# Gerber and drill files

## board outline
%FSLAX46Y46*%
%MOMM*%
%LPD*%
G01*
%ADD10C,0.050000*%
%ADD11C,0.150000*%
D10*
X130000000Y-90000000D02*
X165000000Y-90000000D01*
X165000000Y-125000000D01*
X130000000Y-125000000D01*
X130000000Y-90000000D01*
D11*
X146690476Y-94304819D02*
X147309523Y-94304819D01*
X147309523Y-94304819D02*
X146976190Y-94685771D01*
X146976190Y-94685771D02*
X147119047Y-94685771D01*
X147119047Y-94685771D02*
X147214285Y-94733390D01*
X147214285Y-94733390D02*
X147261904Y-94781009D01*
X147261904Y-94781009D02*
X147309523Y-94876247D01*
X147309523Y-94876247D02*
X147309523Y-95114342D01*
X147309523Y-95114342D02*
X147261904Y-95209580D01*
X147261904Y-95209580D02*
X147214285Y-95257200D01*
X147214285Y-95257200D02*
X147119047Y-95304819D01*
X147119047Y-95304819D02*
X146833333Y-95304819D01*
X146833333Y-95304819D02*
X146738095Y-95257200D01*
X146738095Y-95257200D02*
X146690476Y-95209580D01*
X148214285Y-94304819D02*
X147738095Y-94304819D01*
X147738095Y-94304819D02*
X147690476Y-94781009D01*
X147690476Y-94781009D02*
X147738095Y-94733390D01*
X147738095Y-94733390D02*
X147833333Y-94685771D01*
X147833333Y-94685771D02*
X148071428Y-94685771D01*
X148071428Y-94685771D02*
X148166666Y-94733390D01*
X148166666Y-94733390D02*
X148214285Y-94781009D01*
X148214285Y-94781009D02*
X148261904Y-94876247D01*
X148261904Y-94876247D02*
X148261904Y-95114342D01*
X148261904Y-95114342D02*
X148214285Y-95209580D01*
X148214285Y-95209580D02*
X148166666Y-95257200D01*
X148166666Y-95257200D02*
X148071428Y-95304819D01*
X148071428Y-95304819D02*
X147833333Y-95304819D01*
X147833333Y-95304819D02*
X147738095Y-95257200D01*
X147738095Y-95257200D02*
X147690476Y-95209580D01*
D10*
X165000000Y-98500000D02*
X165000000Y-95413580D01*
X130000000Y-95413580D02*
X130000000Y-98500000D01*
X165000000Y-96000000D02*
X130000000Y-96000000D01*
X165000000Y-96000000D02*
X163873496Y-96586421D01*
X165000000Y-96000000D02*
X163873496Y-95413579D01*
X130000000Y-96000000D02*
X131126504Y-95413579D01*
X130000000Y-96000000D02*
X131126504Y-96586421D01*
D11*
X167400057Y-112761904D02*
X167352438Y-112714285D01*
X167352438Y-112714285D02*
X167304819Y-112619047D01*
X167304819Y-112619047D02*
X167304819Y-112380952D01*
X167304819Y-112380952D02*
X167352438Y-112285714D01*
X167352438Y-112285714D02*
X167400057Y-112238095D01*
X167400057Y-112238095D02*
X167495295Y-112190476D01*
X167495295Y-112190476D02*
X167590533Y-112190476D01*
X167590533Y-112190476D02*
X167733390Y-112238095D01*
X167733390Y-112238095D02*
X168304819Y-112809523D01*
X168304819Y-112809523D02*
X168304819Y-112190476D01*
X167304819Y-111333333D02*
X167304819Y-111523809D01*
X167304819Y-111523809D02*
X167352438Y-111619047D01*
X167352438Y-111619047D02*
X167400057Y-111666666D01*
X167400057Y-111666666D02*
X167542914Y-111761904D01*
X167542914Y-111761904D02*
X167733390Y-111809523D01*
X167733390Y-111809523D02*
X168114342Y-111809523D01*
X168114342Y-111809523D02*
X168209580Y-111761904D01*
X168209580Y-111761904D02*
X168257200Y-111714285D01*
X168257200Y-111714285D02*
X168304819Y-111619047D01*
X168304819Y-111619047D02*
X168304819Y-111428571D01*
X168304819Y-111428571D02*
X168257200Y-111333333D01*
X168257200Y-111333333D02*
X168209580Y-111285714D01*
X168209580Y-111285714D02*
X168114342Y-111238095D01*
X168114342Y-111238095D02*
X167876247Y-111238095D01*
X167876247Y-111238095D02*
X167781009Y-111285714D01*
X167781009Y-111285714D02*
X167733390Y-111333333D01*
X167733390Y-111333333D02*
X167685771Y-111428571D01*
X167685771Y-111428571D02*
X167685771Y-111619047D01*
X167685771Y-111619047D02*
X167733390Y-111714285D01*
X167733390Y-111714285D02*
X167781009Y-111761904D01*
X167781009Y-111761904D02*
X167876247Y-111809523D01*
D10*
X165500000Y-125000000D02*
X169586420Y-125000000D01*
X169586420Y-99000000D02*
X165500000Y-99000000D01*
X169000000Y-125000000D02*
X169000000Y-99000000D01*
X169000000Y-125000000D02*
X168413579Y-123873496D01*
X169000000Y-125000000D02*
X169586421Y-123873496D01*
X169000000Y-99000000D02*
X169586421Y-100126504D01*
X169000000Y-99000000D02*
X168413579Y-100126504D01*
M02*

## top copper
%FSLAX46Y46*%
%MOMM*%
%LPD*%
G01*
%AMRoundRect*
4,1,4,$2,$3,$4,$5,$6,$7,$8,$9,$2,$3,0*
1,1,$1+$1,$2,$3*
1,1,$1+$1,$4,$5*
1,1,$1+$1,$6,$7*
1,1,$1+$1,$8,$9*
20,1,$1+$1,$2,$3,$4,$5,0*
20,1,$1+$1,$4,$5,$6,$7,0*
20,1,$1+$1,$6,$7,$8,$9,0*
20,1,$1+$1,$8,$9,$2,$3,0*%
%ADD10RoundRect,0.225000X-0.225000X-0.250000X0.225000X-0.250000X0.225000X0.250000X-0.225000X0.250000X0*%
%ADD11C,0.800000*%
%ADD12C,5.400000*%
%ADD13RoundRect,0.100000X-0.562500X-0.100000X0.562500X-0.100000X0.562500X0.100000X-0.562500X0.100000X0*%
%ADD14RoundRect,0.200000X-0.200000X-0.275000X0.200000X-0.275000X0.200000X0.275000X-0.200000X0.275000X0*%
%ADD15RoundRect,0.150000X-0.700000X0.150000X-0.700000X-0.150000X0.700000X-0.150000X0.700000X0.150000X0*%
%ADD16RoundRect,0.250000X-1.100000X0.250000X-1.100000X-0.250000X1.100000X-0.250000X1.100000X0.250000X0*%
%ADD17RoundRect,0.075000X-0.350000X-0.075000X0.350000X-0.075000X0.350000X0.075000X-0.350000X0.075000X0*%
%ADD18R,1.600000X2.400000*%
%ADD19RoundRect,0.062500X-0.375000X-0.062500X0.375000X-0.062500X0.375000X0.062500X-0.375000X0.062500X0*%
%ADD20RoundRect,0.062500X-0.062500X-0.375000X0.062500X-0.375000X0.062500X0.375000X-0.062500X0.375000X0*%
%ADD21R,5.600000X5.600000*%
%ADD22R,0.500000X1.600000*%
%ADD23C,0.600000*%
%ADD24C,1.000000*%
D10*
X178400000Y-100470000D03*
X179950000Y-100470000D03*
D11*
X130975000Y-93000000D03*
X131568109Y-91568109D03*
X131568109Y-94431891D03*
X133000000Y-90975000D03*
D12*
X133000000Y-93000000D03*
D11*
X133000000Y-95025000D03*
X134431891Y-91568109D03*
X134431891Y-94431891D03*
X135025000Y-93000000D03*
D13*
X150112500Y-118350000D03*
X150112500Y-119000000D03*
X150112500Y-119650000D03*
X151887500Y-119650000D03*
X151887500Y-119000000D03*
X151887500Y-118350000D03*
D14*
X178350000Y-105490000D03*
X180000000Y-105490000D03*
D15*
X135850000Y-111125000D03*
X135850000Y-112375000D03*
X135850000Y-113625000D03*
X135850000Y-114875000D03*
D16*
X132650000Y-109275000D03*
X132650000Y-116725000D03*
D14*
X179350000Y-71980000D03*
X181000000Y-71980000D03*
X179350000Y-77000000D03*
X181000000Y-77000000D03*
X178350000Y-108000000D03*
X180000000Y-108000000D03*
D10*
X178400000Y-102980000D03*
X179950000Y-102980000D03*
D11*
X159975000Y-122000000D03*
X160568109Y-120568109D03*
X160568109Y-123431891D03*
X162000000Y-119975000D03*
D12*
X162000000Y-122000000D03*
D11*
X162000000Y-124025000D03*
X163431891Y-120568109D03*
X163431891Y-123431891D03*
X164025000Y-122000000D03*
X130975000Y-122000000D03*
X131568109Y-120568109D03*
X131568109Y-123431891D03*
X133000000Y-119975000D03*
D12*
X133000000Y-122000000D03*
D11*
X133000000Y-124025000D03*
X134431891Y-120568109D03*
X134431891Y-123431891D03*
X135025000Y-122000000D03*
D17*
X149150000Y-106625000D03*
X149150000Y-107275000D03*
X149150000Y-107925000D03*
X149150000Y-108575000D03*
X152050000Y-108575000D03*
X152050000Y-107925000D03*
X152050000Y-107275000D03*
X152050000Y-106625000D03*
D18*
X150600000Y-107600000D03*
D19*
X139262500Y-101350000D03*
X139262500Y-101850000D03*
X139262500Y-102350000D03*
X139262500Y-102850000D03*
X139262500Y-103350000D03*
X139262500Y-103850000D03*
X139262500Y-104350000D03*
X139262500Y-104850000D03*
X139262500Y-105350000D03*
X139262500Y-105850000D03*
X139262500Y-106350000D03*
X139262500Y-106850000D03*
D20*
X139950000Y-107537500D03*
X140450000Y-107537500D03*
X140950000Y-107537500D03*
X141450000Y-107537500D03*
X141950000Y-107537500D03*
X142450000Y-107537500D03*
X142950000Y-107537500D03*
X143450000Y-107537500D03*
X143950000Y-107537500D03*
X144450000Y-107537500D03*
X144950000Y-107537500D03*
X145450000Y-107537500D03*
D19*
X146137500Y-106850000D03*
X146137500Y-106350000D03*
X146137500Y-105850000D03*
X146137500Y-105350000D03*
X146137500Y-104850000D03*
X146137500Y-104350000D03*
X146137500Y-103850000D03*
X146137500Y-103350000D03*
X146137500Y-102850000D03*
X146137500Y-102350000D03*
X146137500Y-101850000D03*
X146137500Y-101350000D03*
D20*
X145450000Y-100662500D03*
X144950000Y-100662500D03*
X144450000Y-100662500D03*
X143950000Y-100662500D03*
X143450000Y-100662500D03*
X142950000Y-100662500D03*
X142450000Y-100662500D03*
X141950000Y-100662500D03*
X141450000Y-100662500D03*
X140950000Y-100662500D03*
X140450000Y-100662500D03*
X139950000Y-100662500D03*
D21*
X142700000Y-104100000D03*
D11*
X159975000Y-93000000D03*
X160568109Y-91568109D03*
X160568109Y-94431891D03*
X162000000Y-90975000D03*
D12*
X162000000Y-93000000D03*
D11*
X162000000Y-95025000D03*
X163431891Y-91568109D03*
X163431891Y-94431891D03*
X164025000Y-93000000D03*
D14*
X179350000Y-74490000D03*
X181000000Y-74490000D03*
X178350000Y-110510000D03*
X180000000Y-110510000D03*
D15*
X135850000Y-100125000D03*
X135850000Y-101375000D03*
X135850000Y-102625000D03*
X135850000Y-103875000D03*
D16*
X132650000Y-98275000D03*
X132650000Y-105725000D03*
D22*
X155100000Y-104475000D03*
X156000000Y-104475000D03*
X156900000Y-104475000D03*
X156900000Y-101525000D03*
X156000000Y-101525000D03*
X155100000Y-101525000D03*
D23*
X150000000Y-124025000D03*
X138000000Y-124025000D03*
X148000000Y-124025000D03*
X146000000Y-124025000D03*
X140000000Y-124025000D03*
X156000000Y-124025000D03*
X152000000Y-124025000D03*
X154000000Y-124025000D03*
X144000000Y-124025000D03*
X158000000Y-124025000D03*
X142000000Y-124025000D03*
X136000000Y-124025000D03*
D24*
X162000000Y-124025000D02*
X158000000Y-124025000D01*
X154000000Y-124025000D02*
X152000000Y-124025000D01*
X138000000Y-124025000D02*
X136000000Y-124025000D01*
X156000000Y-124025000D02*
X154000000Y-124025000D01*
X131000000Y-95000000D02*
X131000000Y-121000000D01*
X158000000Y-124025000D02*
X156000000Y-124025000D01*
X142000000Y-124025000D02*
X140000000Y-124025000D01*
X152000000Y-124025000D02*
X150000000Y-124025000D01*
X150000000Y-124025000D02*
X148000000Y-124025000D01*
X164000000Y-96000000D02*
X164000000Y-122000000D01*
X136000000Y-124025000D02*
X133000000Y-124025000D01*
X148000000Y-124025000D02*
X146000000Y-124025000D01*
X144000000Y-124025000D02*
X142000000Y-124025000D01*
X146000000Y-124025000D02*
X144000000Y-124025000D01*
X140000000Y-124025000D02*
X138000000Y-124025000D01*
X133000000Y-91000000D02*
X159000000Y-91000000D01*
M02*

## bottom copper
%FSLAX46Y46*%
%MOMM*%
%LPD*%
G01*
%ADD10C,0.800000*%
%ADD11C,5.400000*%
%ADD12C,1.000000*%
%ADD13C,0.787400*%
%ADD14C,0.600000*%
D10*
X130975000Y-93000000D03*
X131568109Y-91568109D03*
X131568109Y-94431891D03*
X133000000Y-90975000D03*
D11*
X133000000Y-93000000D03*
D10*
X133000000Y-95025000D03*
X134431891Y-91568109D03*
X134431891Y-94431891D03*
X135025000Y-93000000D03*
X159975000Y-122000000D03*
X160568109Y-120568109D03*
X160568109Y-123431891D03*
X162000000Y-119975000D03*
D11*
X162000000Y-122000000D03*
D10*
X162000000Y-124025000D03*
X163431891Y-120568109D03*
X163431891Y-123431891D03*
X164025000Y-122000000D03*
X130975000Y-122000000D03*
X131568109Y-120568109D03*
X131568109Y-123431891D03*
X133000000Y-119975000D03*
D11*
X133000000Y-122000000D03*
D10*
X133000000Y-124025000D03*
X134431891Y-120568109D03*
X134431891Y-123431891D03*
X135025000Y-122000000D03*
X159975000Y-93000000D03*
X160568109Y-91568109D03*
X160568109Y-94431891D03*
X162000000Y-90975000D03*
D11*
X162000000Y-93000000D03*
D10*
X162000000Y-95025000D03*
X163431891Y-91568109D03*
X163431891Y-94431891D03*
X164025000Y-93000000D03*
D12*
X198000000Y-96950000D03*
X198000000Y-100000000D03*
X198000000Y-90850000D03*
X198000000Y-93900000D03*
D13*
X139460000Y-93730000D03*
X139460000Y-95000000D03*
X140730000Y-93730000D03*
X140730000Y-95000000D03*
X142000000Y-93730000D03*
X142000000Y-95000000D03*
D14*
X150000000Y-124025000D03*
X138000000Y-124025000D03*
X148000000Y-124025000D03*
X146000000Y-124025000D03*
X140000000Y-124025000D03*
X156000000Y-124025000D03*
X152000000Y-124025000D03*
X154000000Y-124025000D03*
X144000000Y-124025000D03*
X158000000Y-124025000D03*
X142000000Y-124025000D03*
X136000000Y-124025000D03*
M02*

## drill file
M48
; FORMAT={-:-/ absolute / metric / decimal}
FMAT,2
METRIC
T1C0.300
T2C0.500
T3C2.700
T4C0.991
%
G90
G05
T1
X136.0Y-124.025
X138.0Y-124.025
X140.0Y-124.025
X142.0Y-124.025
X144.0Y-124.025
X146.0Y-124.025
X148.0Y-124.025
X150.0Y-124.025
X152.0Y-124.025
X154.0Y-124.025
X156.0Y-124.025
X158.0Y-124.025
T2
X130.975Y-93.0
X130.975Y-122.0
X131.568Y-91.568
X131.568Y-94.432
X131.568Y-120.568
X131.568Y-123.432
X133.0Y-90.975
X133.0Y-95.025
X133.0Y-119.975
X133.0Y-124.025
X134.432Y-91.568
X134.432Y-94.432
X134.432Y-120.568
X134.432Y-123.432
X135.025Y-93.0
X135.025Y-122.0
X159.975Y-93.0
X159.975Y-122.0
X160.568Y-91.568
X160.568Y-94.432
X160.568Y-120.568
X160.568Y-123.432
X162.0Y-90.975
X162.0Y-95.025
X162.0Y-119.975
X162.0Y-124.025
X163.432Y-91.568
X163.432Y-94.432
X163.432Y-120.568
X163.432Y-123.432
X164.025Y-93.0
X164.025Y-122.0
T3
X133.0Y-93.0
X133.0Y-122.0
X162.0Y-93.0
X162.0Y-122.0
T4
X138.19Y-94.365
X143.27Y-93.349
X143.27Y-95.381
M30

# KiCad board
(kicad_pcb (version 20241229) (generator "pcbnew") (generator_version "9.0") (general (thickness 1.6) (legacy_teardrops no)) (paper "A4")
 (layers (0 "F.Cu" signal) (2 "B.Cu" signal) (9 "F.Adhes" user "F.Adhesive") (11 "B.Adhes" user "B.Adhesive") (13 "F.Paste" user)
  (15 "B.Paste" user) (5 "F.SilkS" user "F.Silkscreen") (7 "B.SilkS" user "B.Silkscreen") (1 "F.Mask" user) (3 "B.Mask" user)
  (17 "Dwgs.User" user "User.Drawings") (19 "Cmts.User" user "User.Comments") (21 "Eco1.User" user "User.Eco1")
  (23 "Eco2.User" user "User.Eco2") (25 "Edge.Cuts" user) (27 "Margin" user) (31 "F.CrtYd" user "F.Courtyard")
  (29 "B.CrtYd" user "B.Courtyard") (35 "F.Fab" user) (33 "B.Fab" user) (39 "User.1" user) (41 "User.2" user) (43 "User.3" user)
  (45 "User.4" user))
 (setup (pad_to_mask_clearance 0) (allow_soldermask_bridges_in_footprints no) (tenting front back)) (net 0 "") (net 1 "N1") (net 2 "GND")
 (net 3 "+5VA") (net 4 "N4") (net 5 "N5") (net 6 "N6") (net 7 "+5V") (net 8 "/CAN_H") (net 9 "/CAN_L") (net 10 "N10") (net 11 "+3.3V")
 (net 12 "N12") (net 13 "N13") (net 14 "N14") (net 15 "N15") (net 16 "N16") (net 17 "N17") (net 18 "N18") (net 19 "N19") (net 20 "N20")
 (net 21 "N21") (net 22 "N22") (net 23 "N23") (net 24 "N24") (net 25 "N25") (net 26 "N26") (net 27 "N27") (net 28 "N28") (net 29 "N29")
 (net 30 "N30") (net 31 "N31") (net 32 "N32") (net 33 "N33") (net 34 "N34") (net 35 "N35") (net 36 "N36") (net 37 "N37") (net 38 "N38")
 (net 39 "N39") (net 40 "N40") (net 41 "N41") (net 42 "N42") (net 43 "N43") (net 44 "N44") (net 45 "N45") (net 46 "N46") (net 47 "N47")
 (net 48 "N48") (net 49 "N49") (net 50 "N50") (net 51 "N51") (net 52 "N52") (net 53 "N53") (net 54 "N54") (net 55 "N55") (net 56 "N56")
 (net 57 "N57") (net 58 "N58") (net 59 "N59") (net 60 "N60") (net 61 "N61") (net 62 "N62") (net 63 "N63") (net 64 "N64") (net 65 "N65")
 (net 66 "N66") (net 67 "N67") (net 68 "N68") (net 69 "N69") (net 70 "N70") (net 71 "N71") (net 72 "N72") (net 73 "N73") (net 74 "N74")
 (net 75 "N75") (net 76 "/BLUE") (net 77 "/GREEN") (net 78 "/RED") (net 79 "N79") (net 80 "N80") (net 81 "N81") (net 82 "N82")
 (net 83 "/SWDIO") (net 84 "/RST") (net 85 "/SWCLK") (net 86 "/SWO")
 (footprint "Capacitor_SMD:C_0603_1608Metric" (layer "F.Cu") (at 179.175 100.47)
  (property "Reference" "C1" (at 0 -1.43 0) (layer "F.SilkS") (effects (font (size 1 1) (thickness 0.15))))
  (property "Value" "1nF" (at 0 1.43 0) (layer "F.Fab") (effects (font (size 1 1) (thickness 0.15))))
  (pad "1" smd roundrect (at -0.775 0) (size 0.9 0.95) (layers "F.Cu" "F.Mask" "F.Paste") (roundrect_rratio 0.25) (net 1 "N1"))
  (pad "2" smd roundrect (at 0.775 0) (size 0.9 0.95) (layers "F.Cu" "F.Mask" "F.Paste") (roundrect_rratio 0.25) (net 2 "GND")))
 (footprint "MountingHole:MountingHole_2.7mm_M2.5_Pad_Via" (layer "F.Cu") (at 133 93)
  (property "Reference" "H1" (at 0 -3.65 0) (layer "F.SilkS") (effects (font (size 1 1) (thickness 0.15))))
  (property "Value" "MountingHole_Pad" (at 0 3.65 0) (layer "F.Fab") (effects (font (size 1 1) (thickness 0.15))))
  (pad "1" thru_hole circle (at -2.025 0) (size 0.8 0.8) (drill 0.5) (layers "*.Cu" "*.Mask") (remove_unused_layers no) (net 1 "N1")
   (zone_connect 2))
  (pad "1" thru_hole circle (at -1.431891 -1.431891) (size 0.8 0.8) (drill 0.5) (layers "*.Cu" "*.Mask") (remove_unused_layers no)
   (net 1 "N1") (zone_connect 2))
  (pad "1" thru_hole circle (at -1.431891 1.431891) (size 0.8 0.8) (drill 0.5) (layers "*.Cu" "*.Mask") (remove_unused_layers no)
   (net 1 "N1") (zone_connect 2))
  (pad "1" thru_hole circle (at 0 -2.025) (size 0.8 0.8) (drill 0.5) (layers "*.Cu" "*.Mask") (remove_unused_layers no) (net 1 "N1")
   (zone_connect 2))
  (pad "1" thru_hole circle (at 0 0) (size 5.4 5.4) (drill 2.7) (layers "*.Cu" "*.Mask") (remove_unused_layers no) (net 1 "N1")
   (zone_connect 2))
  (pad "1" thru_hole circle (at 0 2.025) (size 0.8 0.8) (drill 0.5) (layers "*.Cu" "*.Mask") (remove_unused_layers no) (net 1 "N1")
   (zone_connect 2))
  (pad "1" thru_hole circle (at 1.431891 -1.431891) (size 0.8 0.8) (drill 0.5) (layers "*.Cu" "*.Mask") (remove_unused_layers no)
   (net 1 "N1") (zone_connect 2))
  (pad "1" thru_hole circle (at 1.431891 1.431891) (size 0.8 0.8) (drill 0.5) (layers "*.Cu" "*.Mask") (remove_unused_layers no)
   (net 1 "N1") (zone_connect 2))
  (pad "1" thru_hole circle (at 2.025 0) (size 0.8 0.8) (drill 0.5) (layers "*.Cu" "*.Mask") (remove_unused_layers no) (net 1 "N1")
   (zone_connect 2)))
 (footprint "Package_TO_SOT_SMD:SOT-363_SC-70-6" (layer "F.Cu") (at 151 119)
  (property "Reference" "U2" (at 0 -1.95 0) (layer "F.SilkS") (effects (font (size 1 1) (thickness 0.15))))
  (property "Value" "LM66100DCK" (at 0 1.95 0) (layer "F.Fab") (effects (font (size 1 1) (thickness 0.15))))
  (pad "1" smd roundrect (at -0.8875 -0.65) (size 1.325 0.4) (layers "F.Cu" "F.Mask" "F.Paste") (roundrect_rratio 0.25) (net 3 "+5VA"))
  (pad "2" smd roundrect (at -0.8875 0) (size 1.325 0.4) (layers "F.Cu" "F.Mask" "F.Paste") (roundrect_rratio 0.25) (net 2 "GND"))
  (pad "3" smd roundrect (at -0.8875 0.65) (size 1.325 0.4) (layers "F.Cu" "F.Mask" "F.Paste") (roundrect_rratio 0.25) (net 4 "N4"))
  (pad "4" smd roundrect (at 0.8875 0.65) (size 1.325 0.4) (layers "F.Cu" "F.Mask" "F.Paste") (roundrect_rratio 0.25) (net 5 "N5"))
  (pad "5" smd roundrect (at 0.8875 0) (size 1.325 0.4) (layers "F.Cu" "F.Mask" "F.Paste") (roundrect_rratio 0.25) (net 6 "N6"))
  (pad "6" smd roundrect (at 0.8875 -0.65) (size 1.325 0.4) (layers "F.Cu" "F.Mask" "F.Paste") (roundrect_rratio 0.25) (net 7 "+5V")))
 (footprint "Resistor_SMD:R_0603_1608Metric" (layer "F.Cu") (at 179.175 105.49)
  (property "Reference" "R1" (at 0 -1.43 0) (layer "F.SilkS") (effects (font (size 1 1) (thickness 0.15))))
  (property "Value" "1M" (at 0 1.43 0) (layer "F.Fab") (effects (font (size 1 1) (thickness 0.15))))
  (pad "1" smd roundrect (at -0.825 0) (size 0.8 0.95) (layers "F.Cu" "F.Mask" "F.Paste") (roundrect_rratio 0.25) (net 1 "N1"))
  (pad "2" smd roundrect (at 0.825 0) (size 0.8 0.95) (layers "F.Cu" "F.Mask" "F.Paste") (roundrect_rratio 0.25) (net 2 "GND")))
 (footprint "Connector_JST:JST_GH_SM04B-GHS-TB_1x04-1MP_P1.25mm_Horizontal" (layer "F.Cu") (at 134 113 -90)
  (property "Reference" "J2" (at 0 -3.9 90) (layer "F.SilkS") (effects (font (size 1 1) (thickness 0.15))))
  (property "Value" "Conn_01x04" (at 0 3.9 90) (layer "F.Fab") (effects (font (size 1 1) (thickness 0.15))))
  (pad "1" smd roundrect (at -1.875 -1.85 270) (size 0.6 1.7) (layers "F.Cu" "F.Mask" "F.Paste") (roundrect_rratio 0.25) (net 3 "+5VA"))
  (pad "2" smd roundrect (at -0.625 -1.85 270) (size 0.6 1.7) (layers "F.Cu" "F.Mask" "F.Paste") (roundrect_rratio 0.25) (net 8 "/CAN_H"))
  (pad "3" smd roundrect (at 0.625 -1.85 270) (size 0.6 1.7) (layers "F.Cu" "F.Mask" "F.Paste") (roundrect_rratio 0.25) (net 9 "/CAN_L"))
  (pad "4" smd roundrect (at 1.875 -1.85 270) (size 0.6 1.7) (layers "F.Cu" "F.Mask" "F.Paste") (roundrect_rratio 0.25) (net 2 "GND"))
  (pad "MP" smd roundrect (at -3.725 1.35 270) (size 1 2.7) (layers "F.Cu" "F.Mask" "F.Paste") (roundrect_rratio 0.25))
  (pad "MP" smd roundrect (at 3.725 1.35 270) (size 1 2.7) (layers "F.Cu" "F.Mask" "F.Paste") (roundrect_rratio 0.25)))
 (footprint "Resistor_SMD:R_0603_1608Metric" (layer "F.Cu") (at 180.175 71.98)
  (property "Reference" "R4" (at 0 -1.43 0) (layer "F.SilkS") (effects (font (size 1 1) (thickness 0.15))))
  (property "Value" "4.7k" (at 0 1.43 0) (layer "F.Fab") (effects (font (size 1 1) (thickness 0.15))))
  (pad "1" smd roundrect (at -0.825 0) (size 0.8 0.95) (layers "F.Cu" "F.Mask" "F.Paste") (roundrect_rratio 0.25) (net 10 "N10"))
  (pad "2" smd roundrect (at 0.825 0) (size 0.8 0.95) (layers "F.Cu" "F.Mask" "F.Paste") (roundrect_rratio 0.25) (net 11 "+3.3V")))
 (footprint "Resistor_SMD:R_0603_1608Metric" (layer "F.Cu") (at 180.175 77)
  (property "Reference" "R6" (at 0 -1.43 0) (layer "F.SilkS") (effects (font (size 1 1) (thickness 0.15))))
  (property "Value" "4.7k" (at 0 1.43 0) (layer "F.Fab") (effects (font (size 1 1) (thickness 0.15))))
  (pad "1" smd roundrect (at -0.825 0) (size 0.8 0.95) (layers "F.Cu" "F.Mask" "F.Paste") (roundrect_rratio 0.25) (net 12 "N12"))
  (pad "2" smd roundrect (at 0.825 0) (size 0.8 0.95) (layers "F.Cu" "F.Mask" "F.Paste") (roundrect_rratio 0.25) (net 11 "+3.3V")))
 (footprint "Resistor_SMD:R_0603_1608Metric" (layer "F.Cu") (at 179.175 108)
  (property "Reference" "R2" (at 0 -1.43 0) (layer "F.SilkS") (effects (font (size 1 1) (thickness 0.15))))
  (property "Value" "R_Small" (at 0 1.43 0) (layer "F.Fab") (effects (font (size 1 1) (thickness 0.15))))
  (pad "1" smd roundrect (at -0.825 0) (size 0.8 0.95) (layers "F.Cu" "F.Mask" "F.Paste") (roundrect_rratio 0.25) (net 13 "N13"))
  (pad "2" smd roundrect (at 0.825 0) (size 0.8 0.95) (layers "F.Cu" "F.Mask" "F.Paste") (roundrect_rratio 0.25) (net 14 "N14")))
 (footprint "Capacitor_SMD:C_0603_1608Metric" (layer "F.Cu") (at 179.175 102.98)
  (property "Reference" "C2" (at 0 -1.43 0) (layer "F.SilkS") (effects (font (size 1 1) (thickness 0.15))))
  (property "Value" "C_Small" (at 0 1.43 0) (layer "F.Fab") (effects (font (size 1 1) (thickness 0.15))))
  (pad "1" smd roundrect (at -0.775 0) (size 0.9 0.95) (layers "F.Cu" "F.Mask" "F.Paste") (roundrect_rratio 0.25) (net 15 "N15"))
  (pad "2" smd roundrect (at 0.775 0) (size 0.9 0.95) (layers "F.Cu" "F.Mask" "F.Paste") (roundrect_rratio 0.25) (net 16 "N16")))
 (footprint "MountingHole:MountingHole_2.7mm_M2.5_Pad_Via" (layer "F.Cu") (at 162 122)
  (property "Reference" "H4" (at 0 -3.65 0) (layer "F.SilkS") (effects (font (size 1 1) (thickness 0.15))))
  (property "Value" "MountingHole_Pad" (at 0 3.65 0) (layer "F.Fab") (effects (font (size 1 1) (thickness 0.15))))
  (pad "1" thru_hole circle (at -2.025 0) (size 0.8 0.8) (drill 0.5) (layers "*.Cu" "*.Mask") (remove_unused_layers no) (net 1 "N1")
   (zone_connect 2))
  (pad "1" thru_hole circle (at -1.431891 -1.431891) (size 0.8 0.8) (drill 0.5) (layers "*.Cu" "*.Mask") (remove_unused_layers no)
   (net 1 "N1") (zone_connect 2))
  (pad "1" thru_hole circle (at -1.431891 1.431891) (size 0.8 0.8) (drill 0.5) (layers "*.Cu" "*.Mask") (remove_unused_layers no)
   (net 1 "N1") (zone_connect 2))
  (pad "1" thru_hole circle (at 0 -2.025) (size 0.8 0.8) (drill 0.5) (layers "*.Cu" "*.Mask") (remove_unused_layers no) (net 1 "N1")
   (zone_connect 2))
  (pad "1" thru_hole circle (at 0 0) (size 5.4 5.4) (drill 2.7) (layers "*.Cu" "*.Mask") (remove_unused_layers no) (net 1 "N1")
   (zone_connect 2))
  (pad "1" thru_hole circle (at 0 2.025) (size 0.8 0.8) (drill 0.5) (layers "*.Cu" "*.Mask") (remove_unused_layers no) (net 1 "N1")
   (zone_connect 2))
  (pad "1" thru_hole circle (at 1.431891 -1.431891) (size 0.8 0.8) (drill 0.5) (layers "*.Cu" "*.Mask") (remove_unused_layers no)
   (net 1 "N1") (zone_connect 2))
  (pad "1" thru_hole circle (at 1.431891 1.431891) (size 0.8 0.8) (drill 0.5) (layers "*.Cu" "*.Mask") (remove_unused_layers no)
   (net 1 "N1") (zone_connect 2))
  (pad "1" thru_hole circle (at 2.025 0) (size 0.8 0.8) (drill 0.5) (layers "*.Cu" "*.Mask") (remove_unused_layers no) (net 1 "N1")
   (zone_connect 2)))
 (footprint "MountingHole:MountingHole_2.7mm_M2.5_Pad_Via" (layer "F.Cu") (at 133 122)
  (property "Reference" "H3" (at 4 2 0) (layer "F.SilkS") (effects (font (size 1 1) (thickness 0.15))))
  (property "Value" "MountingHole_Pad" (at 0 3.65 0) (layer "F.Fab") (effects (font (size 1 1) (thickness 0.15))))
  (pad "1" thru_hole circle (at -2.025 0) (size 0.8 0.8) (drill 0.5) (layers "*.Cu" "*.Mask") (remove_unused_layers no) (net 1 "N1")
   (zone_connect 2))
  (pad "1" thru_hole circle (at -1.431891 -1.431891) (size 0.8 0.8) (drill 0.5) (layers "*.Cu" "*.Mask") (remove_unused_layers no)
   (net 1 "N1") (zone_connect 2))
  (pad "1" thru_hole circle (at -1.431891 1.431891) (size 0.8 0.8) (drill 0.5) (layers "*.Cu" "*.Mask") (remove_unused_layers no)
   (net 1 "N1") (zone_connect 2))
  (pad "1" thru_hole circle (at 0 -2.025) (size 0.8 0.8) (drill 0.5) (layers "*.Cu" "*.Mask") (remove_unused_layers no) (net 1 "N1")
   (zone_connect 2))
  (pad "1" thru_hole circle (at 0 0) (size 5.4 5.4) (drill 2.7) (layers "*.Cu" "*.Mask") (remove_unused_layers no) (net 1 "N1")
   (zone_connect 2))
  (pad "1" thru_hole circle (at 0 2.025) (size 0.8 0.8) (drill 0.5) (layers "*.Cu" "*.Mask") (remove_unused_layers no) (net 1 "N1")
   (zone_connect 2))
  (pad "1" thru_hole circle (at 1.431891 -1.431891) (size 0.8 0.8) (drill 0.5) (layers "*.Cu" "*.Mask") (remove_unused_layers no)
   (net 1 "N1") (zone_connect 2))
  (pad "1" thru_hole circle (at 1.431891 1.431891) (size 0.8 0.8) (drill 0.5) (layers "*.Cu" "*.Mask") (remove_unused_layers no)
   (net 1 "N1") (zone_connect 2))
  (pad "1" thru_hole circle (at 2.025 0) (size 0.8 0.8) (drill 0.5) (layers "*.Cu" "*.Mask") (remove_unused_layers no) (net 1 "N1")
   (zone_connect 2)))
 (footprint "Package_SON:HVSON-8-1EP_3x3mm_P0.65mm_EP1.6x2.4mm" (layer "F.Cu") (at 150.6 107.6)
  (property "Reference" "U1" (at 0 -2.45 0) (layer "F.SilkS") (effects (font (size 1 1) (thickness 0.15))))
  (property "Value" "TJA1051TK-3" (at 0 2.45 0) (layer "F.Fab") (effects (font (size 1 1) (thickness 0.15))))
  (pad "" smd roundrect (at -0.4 -0.6) (size 0.64 0.97) (layers "F.Paste") (roundrect_rratio 0.25))
  (pad "" smd roundrect (at -0.4 0.6) (size 0.64 0.97) (layers "F.Paste") (roundrect_rratio 0.25))
  (pad "" smd roundrect (at 0.4 -0.6) (size 0.64 0.97) (layers "F.Paste") (roundrect_rratio 0.25))
  (pad "" smd roundrect (at 0.4 0.6) (size 0.64 0.97) (layers "F.Paste") (roundrect_rratio 0.25))
  (pad "1" smd roundrect (at -1.45 -0.975) (size 0.85 0.3) (layers "F.Cu" "F.Mask" "F.Paste") (roundrect_rratio 0.25) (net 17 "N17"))
  (pad "2" smd roundrect (at -1.45 -0.325) (size 0.85 0.3) (layers "F.Cu" "F.Mask" "F.Paste") (roundrect_rratio 0.25) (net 2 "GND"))
  (pad "3" smd roundrect (at -1.45 0.325) (size 0.85 0.3) (layers "F.Cu" "F.Mask" "F.Paste") (roundrect_rratio 0.25) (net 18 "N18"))
  (pad "4" smd roundrect (at -1.45 0.975) (size 0.85 0.3) (layers "F.Cu" "F.Mask" "F.Paste") (roundrect_rratio 0.25) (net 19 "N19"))
  (pad "5" smd roundrect (at 1.45 0.975) (size 0.85 0.3) (layers "F.Cu" "F.Mask" "F.Paste") (roundrect_rratio 0.25) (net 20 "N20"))
  (pad "6" smd roundrect (at 1.45 0.325) (size 0.85 0.3) (layers "F.Cu" "F.Mask" "F.Paste") (roundrect_rratio 0.25) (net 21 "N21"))
  (pad "7" smd roundrect (at 1.45 -0.325) (size 0.85 0.3) (layers "F.Cu" "F.Mask" "F.Paste") (roundrect_rratio 0.25) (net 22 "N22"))
  (pad "8" smd roundrect (at 1.45 -0.975) (size 0.85 0.3) (layers "F.Cu" "F.Mask" "F.Paste") (roundrect_rratio 0.25) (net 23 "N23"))
  (pad "9" smd rect (at 0 0) (size 1.6 2.4) (layers "F.Cu" "F.Mask") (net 2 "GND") (zone_connect 2)))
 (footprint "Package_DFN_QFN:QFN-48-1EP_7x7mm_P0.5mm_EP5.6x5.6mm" (layer "F.Cu") (at 142.7 104.1)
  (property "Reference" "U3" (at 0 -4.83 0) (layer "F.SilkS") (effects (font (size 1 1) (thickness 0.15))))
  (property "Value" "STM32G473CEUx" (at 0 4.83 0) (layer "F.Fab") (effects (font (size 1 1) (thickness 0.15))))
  (pad "" smd roundrect (at -2.1 -2.1) (size 1.13 1.13) (layers "F.Paste") (roundrect_rratio 0.221239))
  (pad "" smd roundrect (at -2.1 -0.7) (size 1.13 1.13) (layers "F.Paste") (roundrect_rratio 0.221239))
  (pad "" smd roundrect (at -2.1 0.7) (size 1.13 1.13) (layers "F.Paste") (roundrect_rratio 0.221239))
  (pad "" smd roundrect (at -2.1 2.1) (size 1.13 1.13) (layers "F.Paste") (roundrect_rratio 0.221239))
  (pad "" smd roundrect (at -0.7 -2.1) (size 1.13 1.13) (layers "F.Paste") (roundrect_rratio 0.221239))
  (pad "" smd roundrect (at -0.7 -0.7) (size 1.13 1.13) (layers "F.Paste") (roundrect_rratio 0.221239))
  (pad "" smd roundrect (at -0.7 0.7) (size 1.13 1.13) (layers "F.Paste") (roundrect_rratio 0.221239))
  (pad "" smd roundrect (at -0.7 2.1) (size 1.13 1.13) (layers "F.Paste") (roundrect_rratio 0.221239))
  (pad "" smd roundrect (at 0.7 -2.1) (size 1.13 1.13) (layers "F.Paste") (roundrect_rratio 0.221239))
  (pad "" smd roundrect (at 0.7 -0.7) (size 1.13 1.13) (layers "F.Paste") (roundrect_rratio 0.221239))
  (pad "" smd roundrect (at 0.7 0.7) (size 1.13 1.13) (layers "F.Paste") (roundrect_rratio 0.221239))
  (pad "" smd roundrect (at 0.7 2.1) (size 1.13 1.13) (layers "F.Paste") (roundrect_rratio 0.221239))
  (pad "" smd roundrect (at 2.1 -2.1) (size 1.13 1.13) (layers "F.Paste") (roundrect_rratio 0.221239))
  (pad "" smd roundrect (at 2.1 -0.7) (size 1.13 1.13) (layers "F.Paste") (roundrect_rratio 0.221239))
  (pad "" smd roundrect (at 2.1 0.7) (size 1.13 1.13) (layers "F.Paste") (roundrect_rratio 0.221239))
  (pad "" smd roundrect (at 2.1 2.1) (size 1.13 1.13) (layers "F.Paste") (roundrect_rratio 0.221239))
  (pad "1" smd roundrect (at -3.4375 -2.75) (size 0.875 0.25) (layers "F.Cu" "F.Mask" "F.Paste") (roundrect_rratio 0.25) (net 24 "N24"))
  (pad "2" smd roundrect (at -3.4375 -2.25) (size 0.875 0.25) (layers "F.Cu" "F.Mask" "F.Paste") (roundrect_rratio 0.25) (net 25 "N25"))
  (pad "3" smd roundrect (at -3.4375 -1.75) (size 0.875 0.25) (layers "F.Cu" "F.Mask" "F.Paste") (roundrect_rratio 0.25) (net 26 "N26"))
  (pad "4" smd roundrect (at -3.4375 -1.25) (size 0.875 0.25) (layers "F.Cu" "F.Mask" "F.Paste") (roundrect_rratio 0.25) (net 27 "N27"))
  (pad "5" smd roundrect (at -3.4375 -0.75) (size 0.875 0.25) (layers "F.Cu" "F.Mask" "F.Paste") (roundrect_rratio 0.25) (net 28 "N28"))
  (pad "6" smd roundrect (at -3.4375 -0.25) (size 0.875 0.25) (layers "F.Cu" "F.Mask" "F.Paste") (roundrect_rratio 0.25) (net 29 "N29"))
  (pad "7" smd roundrect (at -3.4375 0.25) (size 0.875 0.25) (layers "F.Cu" "F.Mask" "F.Paste") (roundrect_rratio 0.25) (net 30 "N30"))
  (pad "8" smd roundrect (at -3.4375 0.75) (size 0.875 0.25) (layers "F.Cu" "F.Mask" "F.Paste") (roundrect_rratio 0.25) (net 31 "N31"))
  (pad "9" smd roundrect (at -3.4375 1.25) (size 0.875 0.25) (layers "F.Cu" "F.Mask" "F.Paste") (roundrect_rratio 0.25) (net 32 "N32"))
  (pad "10" smd roundrect (at -3.4375 1.75) (size 0.875 0.25) (layers "F.Cu" "F.Mask" "F.Paste") (roundrect_rratio 0.25) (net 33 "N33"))
  (pad "11" smd roundrect (at -3.4375 2.25) (size 0.875 0.25) (layers "F.Cu" "F.Mask" "F.Paste") (roundrect_rratio 0.25) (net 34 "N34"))
  (pad "12" smd roundrect (at -3.4375 2.75) (size 0.875 0.25) (layers "F.Cu" "F.Mask" "F.Paste") (roundrect_rratio 0.25) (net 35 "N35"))
  (pad "13" smd roundrect (at -2.75 3.4375) (size 0.25 0.875) (layers "F.Cu" "F.Mask" "F.Paste") (roundrect_rratio 0.25) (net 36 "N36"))
  (pad "14" smd roundrect (at -2.25 3.4375) (size 0.25 0.875) (layers "F.Cu" "F.Mask" "F.Paste") (roundrect_rratio 0.25) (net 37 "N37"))
  (pad "15" smd roundrect (at -1.75 3.4375) (size 0.25 0.875) (layers "F.Cu" "F.Mask" "F.Paste") (roundrect_rratio 0.25) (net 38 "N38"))
  (pad "16" smd roundrect (at -1.25 3.4375) (size 0.25 0.875) (layers "F.Cu" "F.Mask" "F.Paste") (roundrect_rratio 0.25) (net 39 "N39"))
  (pad "17" smd roundrect (at -0.75 3.4375) (size 0.25 0.875) (layers "F.Cu" "F.Mask" "F.Paste") (roundrect_rratio 0.25) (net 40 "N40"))
  (pad "18" smd roundrect (at -0.25 3.4375) (size 0.25 0.875) (layers "F.Cu" "F.Mask" "F.Paste") (roundrect_rratio 0.25) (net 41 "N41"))
  (pad "19" smd roundrect (at 0.25 3.4375) (size 0.25 0.875) (layers "F.Cu" "F.Mask" "F.Paste") (roundrect_rratio 0.25) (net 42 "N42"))
  (pad "20" smd roundrect (at 0.75 3.4375) (size 0.25 0.875) (layers "F.Cu" "F.Mask" "F.Paste") (roundrect_rratio 0.25) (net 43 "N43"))
  (pad "21" smd roundrect (at 1.25 3.4375) (size 0.25 0.875) (layers "F.Cu" "F.Mask" "F.Paste") (roundrect_rratio 0.25) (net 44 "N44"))
  (pad "22" smd roundrect (at 1.75 3.4375) (size 0.25 0.875) (layers "F.Cu" "F.Mask" "F.Paste") (roundrect_rratio 0.25) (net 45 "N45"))
  (pad "23" smd roundrect (at 2.25 3.4375) (size 0.25 0.875) (layers "F.Cu" "F.Mask" "F.Paste") (roundrect_rratio 0.25) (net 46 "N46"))
  (pad "24" smd roundrect (at 2.75 3.4375) (size 0.25 0.875) (layers "F.Cu" "F.Mask" "F.Paste") (roundrect_rratio 0.25) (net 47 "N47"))
  (pad "25" smd roundrect (at 3.4375 2.75) (size 0.875 0.25) (layers "F.Cu" "F.Mask" "F.Paste") (roundrect_rratio 0.25) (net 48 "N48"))
  (pad "26" smd roundrect (at 3.4375 2.25) (size 0.875 0.25) (layers "F.Cu" "F.Mask" "F.Paste") (roundrect_rratio 0.25) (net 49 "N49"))
  (pad "27" smd roundrect (at 3.4375 1.75) (size 0.875 0.25) (layers "F.Cu" "F.Mask" "F.Paste") (roundrect_rratio 0.25) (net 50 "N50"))
  (pad "28" smd roundrect (at 3.4375 1.25) (size 0.875 0.25) (layers "F.Cu" "F.Mask" "F.Paste") (roundrect_rratio 0.25) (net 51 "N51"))
  (pad "29" smd roundrect (at 3.4375 0.75) (size 0.875 0.25) (layers "F.Cu" "F.Mask" "F.Paste") (roundrect_rratio 0.25) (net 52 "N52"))
  (pad "30" smd roundrect (at 3.4375 0.25) (size 0.875 0.25) (layers "F.Cu" "F.Mask" "F.Paste") (roundrect_rratio 0.25) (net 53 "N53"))
  (pad "31" smd roundrect (at 3.4375 -0.25) (size 0.875 0.25) (layers "F.Cu" "F.Mask" "F.Paste") (roundrect_rratio 0.25) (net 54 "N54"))
  (pad "32" smd roundrect (at 3.4375 -0.75) (size 0.875 0.25) (layers "F.Cu" "F.Mask" "F.Paste") (roundrect_rratio 0.25) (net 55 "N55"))
  (pad "33" smd roundrect (at 3.4375 -1.25) (size 0.875 0.25) (layers "F.Cu" "F.Mask" "F.Paste") (roundrect_rratio 0.25) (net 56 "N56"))
  (pad "34" smd roundrect (at 3.4375 -1.75) (size 0.875 0.25) (layers "F.Cu" "F.Mask" "F.Paste") (roundrect_rratio 0.25) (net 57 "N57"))
  (pad "35" smd roundrect (at 3.4375 -2.25) (size 0.875 0.25) (layers "F.Cu" "F.Mask" "F.Paste") (roundrect_rratio 0.25) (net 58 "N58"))
  (pad "36" smd roundrect (at 3.4375 -2.75) (size 0.875 0.25) (layers "F.Cu" "F.Mask" "F.Paste") (roundrect_rratio 0.25) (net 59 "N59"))
  (pad "37" smd roundrect (at 2.75 -3.4375) (size 0.25 0.875) (layers "F.Cu" "F.Mask" "F.Paste") (roundrect_rratio 0.25) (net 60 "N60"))
  (pad "38" smd roundrect (at 2.25 -3.4375) (size 0.25 0.875) (layers "F.Cu" "F.Mask" "F.Paste") (roundrect_rratio 0.25) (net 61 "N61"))
  (pad "39" smd roundrect (at 1.75 -3.4375) (size 0.25 0.875) (layers "F.Cu" "F.Mask" "F.Paste") (roundrect_rratio 0.25) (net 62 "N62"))
  (pad "40" smd roundrect (at 1.25 -3.4375) (size 0.25 0.875) (layers "F.Cu" "F.Mask" "F.Paste") (roundrect_rratio 0.25) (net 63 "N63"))
  (pad "41" smd roundrect (at 0.75 -3.4375) (size 0.25 0.875) (layers "F.Cu" "F.Mask" "F.Paste") (roundrect_rratio 0.25) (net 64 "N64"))
  (pad "42" smd roundrect (at 0.25 -3.4375) (size 0.25 0.875) (layers "F.Cu" "F.Mask" "F.Paste") (roundrect_rratio 0.25) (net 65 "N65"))
  (pad "43" smd roundrect (at -0.25 -3.4375) (size 0.25 0.875) (layers "F.Cu" "F.Mask" "F.Paste") (roundrect_rratio 0.25) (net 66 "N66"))
  (pad "44" smd roundrect (at -0.75 -3.4375) (size 0.25 0.875) (layers "F.Cu" "F.Mask" "F.Paste") (roundrect_rratio 0.25) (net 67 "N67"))
  (pad "45" smd roundrect (at -1.25 -3.4375) (size 0.25 0.875) (layers "F.Cu" "F.Mask" "F.Paste") (roundrect_rratio 0.25) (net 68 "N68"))
  (pad "46" smd roundrect (at -1.75 -3.4375) (size 0.25 0.875) (layers "F.Cu" "F.Mask" "F.Paste") (roundrect_rratio 0.25) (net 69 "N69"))
  (pad "47" smd roundrect (at -2.25 -3.4375) (size 0.25 0.875) (layers "F.Cu" "F.Mask" "F.Paste") (roundrect_rratio 0.25) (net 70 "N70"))
  (pad "48" smd roundrect (at -2.75 -3.4375) (size 0.25 0.875) (layers "F.Cu" "F.Mask" "F.Paste") (roundrect_rratio 0.25) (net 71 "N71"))
  (pad "49" smd rect (at 0 0) (size 5.6 5.6) (layers "F.Cu" "F.Mask") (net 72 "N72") (zone_connect 2)))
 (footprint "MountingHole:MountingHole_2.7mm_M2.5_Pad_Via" (layer "F.Cu") (at 162 93)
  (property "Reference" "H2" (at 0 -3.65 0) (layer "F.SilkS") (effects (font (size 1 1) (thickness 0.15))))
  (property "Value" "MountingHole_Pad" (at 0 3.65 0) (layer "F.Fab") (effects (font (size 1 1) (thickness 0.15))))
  (pad "1" thru_hole circle (at -2.025 0) (size 0.8 0.8) (drill 0.5) (layers "*.Cu" "*.Mask") (remove_unused_layers no) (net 1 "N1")
   (zone_connect 2))
  (pad "1" thru_hole circle (at -1.431891 -1.431891) (size 0.8 0.8) (drill 0.5) (layers "*.Cu" "*.Mask") (remove_unused_layers no)
   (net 1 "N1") (zone_connect 2))
  (pad "1" thru_hole circle (at -1.431891 1.431891) (size 0.8 0.8) (drill 0.5) (layers "*.Cu" "*.Mask") (remove_unused_layers no)
   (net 1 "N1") (zone_connect 2))
  (pad "1" thru_hole circle (at 0 -2.025) (size 0.8 0.8) (drill 0.5) (layers "*.Cu" "*.Mask") (remove_unused_layers no) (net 1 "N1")
   (zone_connect 2))
  (pad "1" thru_hole circle (at 0 0) (size 5.4 5.4) (drill 2.7) (layers "*.Cu" "*.Mask") (remove_unused_layers no) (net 1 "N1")
   (zone_connect 2))
  (pad "1" thru_hole circle (at 0 2.025) (size 0.8 0.8) (drill 0.5) (layers "*.Cu" "*.Mask") (remove_unused_layers no) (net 1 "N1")
   (zone_connect 2))
  (pad "1" thru_hole circle (at 1.431891 -1.431891) (size 0.8 0.8) (drill 0.5) (layers "*.Cu" "*.Mask") (remove_unused_layers no)
   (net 1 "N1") (zone_connect 2))
  (pad "1" thru_hole circle (at 1.431891 1.431891) (size 0.8 0.8) (drill 0.5) (layers "*.Cu" "*.Mask") (remove_unused_layers no)
   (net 1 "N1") (zone_connect 2))
  (pad "1" thru_hole circle (at 2.025 0) (size 0.8 0.8) (drill 0.5) (layers "*.Cu" "*.Mask") (remove_unused_layers no) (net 1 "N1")
   (zone_connect 2)))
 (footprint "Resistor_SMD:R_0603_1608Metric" (layer "F.Cu") (at 180.175 74.49)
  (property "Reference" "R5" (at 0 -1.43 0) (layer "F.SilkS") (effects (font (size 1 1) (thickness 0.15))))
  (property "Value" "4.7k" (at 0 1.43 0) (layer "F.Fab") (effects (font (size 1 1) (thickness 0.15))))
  (pad "1" smd roundrect (at -0.825 0) (size 0.8 0.95) (layers "F.Cu" "F.Mask" "F.Paste") (roundrect_rratio 0.25) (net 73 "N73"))
  (pad "2" smd roundrect (at 0.825 0) (size 0.8 0.95) (layers "F.Cu" "F.Mask" "F.Paste") (roundrect_rratio 0.25) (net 11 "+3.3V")))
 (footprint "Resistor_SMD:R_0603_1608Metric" (layer "F.Cu") (at 179.175 110.51)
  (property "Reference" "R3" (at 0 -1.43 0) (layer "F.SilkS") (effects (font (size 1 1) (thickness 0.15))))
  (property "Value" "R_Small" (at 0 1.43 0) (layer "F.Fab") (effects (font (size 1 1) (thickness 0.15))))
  (pad "1" smd roundrect (at -0.825 0) (size 0.8 0.95) (layers "F.Cu" "F.Mask" "F.Paste") (roundrect_rratio 0.25) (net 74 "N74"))
  (pad "2" smd roundrect (at 0.825 0) (size 0.8 0.95) (layers "F.Cu" "F.Mask" "F.Paste") (roundrect_rratio 0.25) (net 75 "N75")))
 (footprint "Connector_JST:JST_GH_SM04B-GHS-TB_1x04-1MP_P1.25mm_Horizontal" (layer "F.Cu") (at 134 102 -90)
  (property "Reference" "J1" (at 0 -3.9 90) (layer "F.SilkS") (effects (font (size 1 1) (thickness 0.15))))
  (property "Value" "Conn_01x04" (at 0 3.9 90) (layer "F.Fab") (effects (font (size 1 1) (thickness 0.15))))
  (pad "1" smd roundrect (at -1.875 -1.85 270) (size 0.6 1.7) (layers "F.Cu" "F.Mask" "F.Paste") (roundrect_rratio 0.25) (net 3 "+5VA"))
  (pad "2" smd roundrect (at -0.625 -1.85 270) (size 0.6 1.7) (layers "F.Cu" "F.Mask" "F.Paste") (roundrect_rratio 0.25) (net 8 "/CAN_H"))
  (pad "3" smd roundrect (at 0.625 -1.85 270) (size 0.6 1.7) (layers "F.Cu" "F.Mask" "F.Paste") (roundrect_rratio 0.25) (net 9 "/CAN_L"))
  (pad "4" smd roundrect (at 1.875 -1.85 270) (size 0.6 1.7) (layers "F.Cu" "F.Mask" "F.Paste") (roundrect_rratio 0.25) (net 2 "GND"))
  (pad "MP" smd roundrect (at -3.725 1.35 270) (size 1 2.7) (layers "F.Cu" "F.Mask" "F.Paste") (roundrect_rratio 0.25))
  (pad "MP" smd roundrect (at 3.725 1.35 270) (size 1 2.7) (layers "F.Cu" "F.Mask" "F.Paste") (roundrect_rratio 0.25)))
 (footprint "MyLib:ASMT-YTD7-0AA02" (layer "F.Cu") (at 156 103 90)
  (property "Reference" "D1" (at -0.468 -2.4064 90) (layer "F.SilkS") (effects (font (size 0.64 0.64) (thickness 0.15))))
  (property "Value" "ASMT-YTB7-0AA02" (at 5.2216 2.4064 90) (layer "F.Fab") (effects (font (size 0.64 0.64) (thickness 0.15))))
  (pad "1" smd rect (at -1.475 -0.9 180) (size 0.5 1.6) (layers "F.Cu" "F.Mask" "F.Paste") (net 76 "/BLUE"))
  (pad "2" smd rect (at -1.475 0 180) (size 0.5 1.6) (layers "F.Cu" "F.Mask" "F.Paste") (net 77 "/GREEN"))
  (pad "3" smd rect (at -1.475 0.9 180) (size 0.5 1.6) (layers "F.Cu" "F.Mask" "F.Paste") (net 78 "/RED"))
  (pad "4" smd rect (at 1.475 0.9 180) (size 0.5 1.6) (layers "F.Cu" "F.Mask" "F.Paste") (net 12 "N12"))
  (pad "5" smd rect (at 1.475 0 180) (size 0.5 1.6) (layers "F.Cu" "F.Mask" "F.Paste") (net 73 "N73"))
  (pad "6" smd rect (at 1.475 -0.9 180) (size 0.5 1.6) (layers "F.Cu" "F.Mask" "F.Paste") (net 10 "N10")))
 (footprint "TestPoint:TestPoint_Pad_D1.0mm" (layer "B.Cu") (at 198 96.95 180)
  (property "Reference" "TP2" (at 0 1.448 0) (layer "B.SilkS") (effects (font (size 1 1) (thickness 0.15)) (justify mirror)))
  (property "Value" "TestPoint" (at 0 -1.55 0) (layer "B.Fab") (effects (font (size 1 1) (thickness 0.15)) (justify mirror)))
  (pad "1" smd circle (at 0 0 180) (size 1 1) (layers "B.Cu" "B.Mask") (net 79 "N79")))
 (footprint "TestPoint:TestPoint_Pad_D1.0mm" (layer "B.Cu") (at 198 100 180)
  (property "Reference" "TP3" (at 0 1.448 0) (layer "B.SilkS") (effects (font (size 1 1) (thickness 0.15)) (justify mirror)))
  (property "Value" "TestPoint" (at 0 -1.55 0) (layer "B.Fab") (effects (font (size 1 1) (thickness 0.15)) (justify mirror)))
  (pad "1" smd circle (at 0 0 180) (size 1 1) (layers "B.Cu" "B.Mask") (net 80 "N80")))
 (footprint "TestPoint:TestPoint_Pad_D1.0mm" (layer "B.Cu") (at 198 90.85 180)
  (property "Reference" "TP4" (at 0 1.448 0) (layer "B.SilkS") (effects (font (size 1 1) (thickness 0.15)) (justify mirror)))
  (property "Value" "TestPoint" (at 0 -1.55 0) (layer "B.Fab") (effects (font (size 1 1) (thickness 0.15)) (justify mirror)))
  (pad "1" smd circle (at 0 0 180) (size 1 1) (layers "B.Cu" "B.Mask") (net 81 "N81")))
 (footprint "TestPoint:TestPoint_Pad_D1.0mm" (layer "B.Cu") (at 198 93.9 180)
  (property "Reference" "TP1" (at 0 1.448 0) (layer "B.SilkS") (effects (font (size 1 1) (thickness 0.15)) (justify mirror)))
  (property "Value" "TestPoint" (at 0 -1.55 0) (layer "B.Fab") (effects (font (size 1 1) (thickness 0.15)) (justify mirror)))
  (pad "1" smd circle (at 0 0 180) (size 1 1) (layers "B.Cu" "B.Mask") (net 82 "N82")))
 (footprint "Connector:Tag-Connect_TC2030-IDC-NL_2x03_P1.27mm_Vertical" (layer "B.Cu") (at 140.73 94.365)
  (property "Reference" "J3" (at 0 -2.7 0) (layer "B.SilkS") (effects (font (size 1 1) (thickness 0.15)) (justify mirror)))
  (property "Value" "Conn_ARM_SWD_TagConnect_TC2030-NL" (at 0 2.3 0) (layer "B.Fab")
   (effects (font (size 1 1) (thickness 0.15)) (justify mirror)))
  (pad "" np_thru_hole circle (at -2.54 0) (size 0.9906 0.9906) (drill 0.9906) (layers "*.Cu" "*.Mask"))
  (pad "" np_thru_hole circle (at 2.54 -1.016) (size 0.9906 0.9906) (drill 0.9906) (layers "*.Cu" "*.Mask"))
  (pad "" np_thru_hole circle (at 2.54 1.016) (size 0.9906 0.9906) (drill 0.9906) (layers "*.Cu" "*.Mask"))
  (pad "1" connect circle (at -1.27 -0.635) (size 0.7874 0.7874) (layers "B.Cu" "B.Mask") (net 11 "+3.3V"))
  (pad "2" connect circle (at -1.27 0.635) (size 0.7874 0.7874) (layers "B.Cu" "B.Mask") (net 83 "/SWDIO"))
  (pad "3" connect circle (at 0 -0.635) (size 0.7874 0.7874) (layers "B.Cu" "B.Mask") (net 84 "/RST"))
  (pad "4" connect circle (at 0 0.635) (size 0.7874 0.7874) (layers "B.Cu" "B.Mask") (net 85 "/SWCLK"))
  (pad "5" connect circle (at 1.27 -0.635) (size 0.7874 0.7874) (layers "B.Cu" "B.Mask") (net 2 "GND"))
  (pad "6" connect circle (at 1.27 0.635) (size 0.7874 0.7874) (layers "B.Cu" "B.Mask") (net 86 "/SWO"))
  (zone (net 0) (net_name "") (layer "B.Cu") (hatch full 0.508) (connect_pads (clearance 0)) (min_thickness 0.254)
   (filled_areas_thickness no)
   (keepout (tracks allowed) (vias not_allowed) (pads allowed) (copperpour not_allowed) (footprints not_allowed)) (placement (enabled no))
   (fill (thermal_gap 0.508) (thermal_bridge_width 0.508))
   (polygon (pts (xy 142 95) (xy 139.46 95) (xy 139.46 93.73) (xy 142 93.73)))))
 (gr_rect (start 130 90) (end 165 125) (stroke (width 0.05) (type default)) (fill no) (layer "Edge.Cuts"))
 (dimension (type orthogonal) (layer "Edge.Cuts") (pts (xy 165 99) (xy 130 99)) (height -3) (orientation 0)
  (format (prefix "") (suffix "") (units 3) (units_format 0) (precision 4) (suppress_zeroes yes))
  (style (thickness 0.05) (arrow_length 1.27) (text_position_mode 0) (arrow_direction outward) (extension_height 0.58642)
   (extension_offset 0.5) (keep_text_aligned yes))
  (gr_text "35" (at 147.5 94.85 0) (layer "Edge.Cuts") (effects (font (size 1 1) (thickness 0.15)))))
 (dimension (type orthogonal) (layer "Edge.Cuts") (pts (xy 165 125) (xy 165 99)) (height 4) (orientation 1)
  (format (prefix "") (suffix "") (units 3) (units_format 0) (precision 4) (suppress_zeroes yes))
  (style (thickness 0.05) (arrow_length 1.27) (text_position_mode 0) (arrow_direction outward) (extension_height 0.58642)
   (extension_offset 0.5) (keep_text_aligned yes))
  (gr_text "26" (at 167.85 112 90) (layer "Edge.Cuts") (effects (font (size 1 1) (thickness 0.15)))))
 (segment (start 162 124.025) (end 158 124.025) (width 1) (layers "F.Cu" "F.Mask") (solder_mask_margin 0) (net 1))
 (segment (start 154 124.025) (end 152 124.025) (width 1) (layers "F.Cu" "F.Mask") (solder_mask_margin 0) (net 1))
 (segment (start 138 124.025) (end 136 124.025) (width 1) (layers "F.Cu" "F.Mask") (solder_mask_margin 0) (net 1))
 (segment (start 156 124.025) (end 154 124.025) (width 1) (layers "F.Cu" "F.Mask") (solder_mask_margin 0) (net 1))
 (segment (start 131 95) (end 131 121) (width 1) (layers "F.Cu" "F.Mask") (solder_mask_margin 0) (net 1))
 (segment (start 158 124.025) (end 156 124.025) (width 1) (layers "F.Cu" "F.Mask") (solder_mask_margin 0) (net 1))
 (segment (start 142 124.025) (end 140 124.025) (width 1) (layers "F.Cu" "F.Mask") (solder_mask_margin 0) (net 1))
 (segment (start 152 124.025) (end 150 124.025) (width 1) (layers "F.Cu" "F.Mask") (solder_mask_margin 0) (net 1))
 (segment (start 150 124.025) (end 148 124.025) (width 1) (layers "F.Cu" "F.Mask") (solder_mask_margin 0) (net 1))
 (segment (start 164 96) (end 164 122) (width 1) (layers "F.Cu" "F.Mask") (solder_mask_margin 0) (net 1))
 (segment (start 136 124.025) (end 133 124.025) (width 1) (layers "F.Cu" "F.Mask") (solder_mask_margin 0) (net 1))
 (segment (start 148 124.025) (end 146 124.025) (width 1) (layers "F.Cu" "F.Mask") (solder_mask_margin 0) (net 1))
 (segment (start 144 124.025) (end 142 124.025) (width 1) (layers "F.Cu" "F.Mask") (solder_mask_margin 0) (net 1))
 (segment (start 146 124.025) (end 144 124.025) (width 1) (layers "F.Cu" "F.Mask") (solder_mask_margin 0) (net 1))
 (segment (start 140 124.025) (end 138 124.025) (width 1) (layers "F.Cu" "F.Mask") (solder_mask_margin 0) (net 1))
 (segment (start 133 91) (end 159 91) (width 1) (layers "F.Cu" "F.Mask") (solder_mask_margin 0) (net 1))
 (via (at 150 124.025) (size 0.6) (drill 0.3) (layers "F.Cu" "B.Cu") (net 1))
 (via (at 138 124.025) (size 0.6) (drill 0.3) (layers "F.Cu" "B.Cu") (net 1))
 (via (at 148 124.025) (size 0.6) (drill 0.3) (layers "F.Cu" "B.Cu") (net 1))
 (via (at 146 124.025) (size 0.6) (drill 0.3) (layers "F.Cu" "B.Cu") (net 1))
 (via (at 140 124.025) (size 0.6) (drill 0.3) (layers "F.Cu" "B.Cu") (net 1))
 (via (at 156 124.025) (size 0.6) (drill 0.3) (layers "F.Cu" "B.Cu") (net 1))
 (via (at 152 124.025) (size 0.6) (drill 0.3) (layers "F.Cu" "B.Cu") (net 1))
 (via (at 154 124.025) (size 0.6) (drill 0.3) (layers "F.Cu" "B.Cu") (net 1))
 (via (at 144 124.025) (size 0.6) (drill 0.3) (layers "F.Cu" "B.Cu") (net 1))
 (via (at 158 124.025) (size 0.6) (drill 0.3) (layers "F.Cu" "B.Cu") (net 1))
 (via (at 142 124.025) (size 0.6) (drill 0.3) (layers "F.Cu" "B.Cu") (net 1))
 (via (at 136 124.025) (size 0.6) (drill 0.3) (layers "F.Cu" "B.Cu") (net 1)))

